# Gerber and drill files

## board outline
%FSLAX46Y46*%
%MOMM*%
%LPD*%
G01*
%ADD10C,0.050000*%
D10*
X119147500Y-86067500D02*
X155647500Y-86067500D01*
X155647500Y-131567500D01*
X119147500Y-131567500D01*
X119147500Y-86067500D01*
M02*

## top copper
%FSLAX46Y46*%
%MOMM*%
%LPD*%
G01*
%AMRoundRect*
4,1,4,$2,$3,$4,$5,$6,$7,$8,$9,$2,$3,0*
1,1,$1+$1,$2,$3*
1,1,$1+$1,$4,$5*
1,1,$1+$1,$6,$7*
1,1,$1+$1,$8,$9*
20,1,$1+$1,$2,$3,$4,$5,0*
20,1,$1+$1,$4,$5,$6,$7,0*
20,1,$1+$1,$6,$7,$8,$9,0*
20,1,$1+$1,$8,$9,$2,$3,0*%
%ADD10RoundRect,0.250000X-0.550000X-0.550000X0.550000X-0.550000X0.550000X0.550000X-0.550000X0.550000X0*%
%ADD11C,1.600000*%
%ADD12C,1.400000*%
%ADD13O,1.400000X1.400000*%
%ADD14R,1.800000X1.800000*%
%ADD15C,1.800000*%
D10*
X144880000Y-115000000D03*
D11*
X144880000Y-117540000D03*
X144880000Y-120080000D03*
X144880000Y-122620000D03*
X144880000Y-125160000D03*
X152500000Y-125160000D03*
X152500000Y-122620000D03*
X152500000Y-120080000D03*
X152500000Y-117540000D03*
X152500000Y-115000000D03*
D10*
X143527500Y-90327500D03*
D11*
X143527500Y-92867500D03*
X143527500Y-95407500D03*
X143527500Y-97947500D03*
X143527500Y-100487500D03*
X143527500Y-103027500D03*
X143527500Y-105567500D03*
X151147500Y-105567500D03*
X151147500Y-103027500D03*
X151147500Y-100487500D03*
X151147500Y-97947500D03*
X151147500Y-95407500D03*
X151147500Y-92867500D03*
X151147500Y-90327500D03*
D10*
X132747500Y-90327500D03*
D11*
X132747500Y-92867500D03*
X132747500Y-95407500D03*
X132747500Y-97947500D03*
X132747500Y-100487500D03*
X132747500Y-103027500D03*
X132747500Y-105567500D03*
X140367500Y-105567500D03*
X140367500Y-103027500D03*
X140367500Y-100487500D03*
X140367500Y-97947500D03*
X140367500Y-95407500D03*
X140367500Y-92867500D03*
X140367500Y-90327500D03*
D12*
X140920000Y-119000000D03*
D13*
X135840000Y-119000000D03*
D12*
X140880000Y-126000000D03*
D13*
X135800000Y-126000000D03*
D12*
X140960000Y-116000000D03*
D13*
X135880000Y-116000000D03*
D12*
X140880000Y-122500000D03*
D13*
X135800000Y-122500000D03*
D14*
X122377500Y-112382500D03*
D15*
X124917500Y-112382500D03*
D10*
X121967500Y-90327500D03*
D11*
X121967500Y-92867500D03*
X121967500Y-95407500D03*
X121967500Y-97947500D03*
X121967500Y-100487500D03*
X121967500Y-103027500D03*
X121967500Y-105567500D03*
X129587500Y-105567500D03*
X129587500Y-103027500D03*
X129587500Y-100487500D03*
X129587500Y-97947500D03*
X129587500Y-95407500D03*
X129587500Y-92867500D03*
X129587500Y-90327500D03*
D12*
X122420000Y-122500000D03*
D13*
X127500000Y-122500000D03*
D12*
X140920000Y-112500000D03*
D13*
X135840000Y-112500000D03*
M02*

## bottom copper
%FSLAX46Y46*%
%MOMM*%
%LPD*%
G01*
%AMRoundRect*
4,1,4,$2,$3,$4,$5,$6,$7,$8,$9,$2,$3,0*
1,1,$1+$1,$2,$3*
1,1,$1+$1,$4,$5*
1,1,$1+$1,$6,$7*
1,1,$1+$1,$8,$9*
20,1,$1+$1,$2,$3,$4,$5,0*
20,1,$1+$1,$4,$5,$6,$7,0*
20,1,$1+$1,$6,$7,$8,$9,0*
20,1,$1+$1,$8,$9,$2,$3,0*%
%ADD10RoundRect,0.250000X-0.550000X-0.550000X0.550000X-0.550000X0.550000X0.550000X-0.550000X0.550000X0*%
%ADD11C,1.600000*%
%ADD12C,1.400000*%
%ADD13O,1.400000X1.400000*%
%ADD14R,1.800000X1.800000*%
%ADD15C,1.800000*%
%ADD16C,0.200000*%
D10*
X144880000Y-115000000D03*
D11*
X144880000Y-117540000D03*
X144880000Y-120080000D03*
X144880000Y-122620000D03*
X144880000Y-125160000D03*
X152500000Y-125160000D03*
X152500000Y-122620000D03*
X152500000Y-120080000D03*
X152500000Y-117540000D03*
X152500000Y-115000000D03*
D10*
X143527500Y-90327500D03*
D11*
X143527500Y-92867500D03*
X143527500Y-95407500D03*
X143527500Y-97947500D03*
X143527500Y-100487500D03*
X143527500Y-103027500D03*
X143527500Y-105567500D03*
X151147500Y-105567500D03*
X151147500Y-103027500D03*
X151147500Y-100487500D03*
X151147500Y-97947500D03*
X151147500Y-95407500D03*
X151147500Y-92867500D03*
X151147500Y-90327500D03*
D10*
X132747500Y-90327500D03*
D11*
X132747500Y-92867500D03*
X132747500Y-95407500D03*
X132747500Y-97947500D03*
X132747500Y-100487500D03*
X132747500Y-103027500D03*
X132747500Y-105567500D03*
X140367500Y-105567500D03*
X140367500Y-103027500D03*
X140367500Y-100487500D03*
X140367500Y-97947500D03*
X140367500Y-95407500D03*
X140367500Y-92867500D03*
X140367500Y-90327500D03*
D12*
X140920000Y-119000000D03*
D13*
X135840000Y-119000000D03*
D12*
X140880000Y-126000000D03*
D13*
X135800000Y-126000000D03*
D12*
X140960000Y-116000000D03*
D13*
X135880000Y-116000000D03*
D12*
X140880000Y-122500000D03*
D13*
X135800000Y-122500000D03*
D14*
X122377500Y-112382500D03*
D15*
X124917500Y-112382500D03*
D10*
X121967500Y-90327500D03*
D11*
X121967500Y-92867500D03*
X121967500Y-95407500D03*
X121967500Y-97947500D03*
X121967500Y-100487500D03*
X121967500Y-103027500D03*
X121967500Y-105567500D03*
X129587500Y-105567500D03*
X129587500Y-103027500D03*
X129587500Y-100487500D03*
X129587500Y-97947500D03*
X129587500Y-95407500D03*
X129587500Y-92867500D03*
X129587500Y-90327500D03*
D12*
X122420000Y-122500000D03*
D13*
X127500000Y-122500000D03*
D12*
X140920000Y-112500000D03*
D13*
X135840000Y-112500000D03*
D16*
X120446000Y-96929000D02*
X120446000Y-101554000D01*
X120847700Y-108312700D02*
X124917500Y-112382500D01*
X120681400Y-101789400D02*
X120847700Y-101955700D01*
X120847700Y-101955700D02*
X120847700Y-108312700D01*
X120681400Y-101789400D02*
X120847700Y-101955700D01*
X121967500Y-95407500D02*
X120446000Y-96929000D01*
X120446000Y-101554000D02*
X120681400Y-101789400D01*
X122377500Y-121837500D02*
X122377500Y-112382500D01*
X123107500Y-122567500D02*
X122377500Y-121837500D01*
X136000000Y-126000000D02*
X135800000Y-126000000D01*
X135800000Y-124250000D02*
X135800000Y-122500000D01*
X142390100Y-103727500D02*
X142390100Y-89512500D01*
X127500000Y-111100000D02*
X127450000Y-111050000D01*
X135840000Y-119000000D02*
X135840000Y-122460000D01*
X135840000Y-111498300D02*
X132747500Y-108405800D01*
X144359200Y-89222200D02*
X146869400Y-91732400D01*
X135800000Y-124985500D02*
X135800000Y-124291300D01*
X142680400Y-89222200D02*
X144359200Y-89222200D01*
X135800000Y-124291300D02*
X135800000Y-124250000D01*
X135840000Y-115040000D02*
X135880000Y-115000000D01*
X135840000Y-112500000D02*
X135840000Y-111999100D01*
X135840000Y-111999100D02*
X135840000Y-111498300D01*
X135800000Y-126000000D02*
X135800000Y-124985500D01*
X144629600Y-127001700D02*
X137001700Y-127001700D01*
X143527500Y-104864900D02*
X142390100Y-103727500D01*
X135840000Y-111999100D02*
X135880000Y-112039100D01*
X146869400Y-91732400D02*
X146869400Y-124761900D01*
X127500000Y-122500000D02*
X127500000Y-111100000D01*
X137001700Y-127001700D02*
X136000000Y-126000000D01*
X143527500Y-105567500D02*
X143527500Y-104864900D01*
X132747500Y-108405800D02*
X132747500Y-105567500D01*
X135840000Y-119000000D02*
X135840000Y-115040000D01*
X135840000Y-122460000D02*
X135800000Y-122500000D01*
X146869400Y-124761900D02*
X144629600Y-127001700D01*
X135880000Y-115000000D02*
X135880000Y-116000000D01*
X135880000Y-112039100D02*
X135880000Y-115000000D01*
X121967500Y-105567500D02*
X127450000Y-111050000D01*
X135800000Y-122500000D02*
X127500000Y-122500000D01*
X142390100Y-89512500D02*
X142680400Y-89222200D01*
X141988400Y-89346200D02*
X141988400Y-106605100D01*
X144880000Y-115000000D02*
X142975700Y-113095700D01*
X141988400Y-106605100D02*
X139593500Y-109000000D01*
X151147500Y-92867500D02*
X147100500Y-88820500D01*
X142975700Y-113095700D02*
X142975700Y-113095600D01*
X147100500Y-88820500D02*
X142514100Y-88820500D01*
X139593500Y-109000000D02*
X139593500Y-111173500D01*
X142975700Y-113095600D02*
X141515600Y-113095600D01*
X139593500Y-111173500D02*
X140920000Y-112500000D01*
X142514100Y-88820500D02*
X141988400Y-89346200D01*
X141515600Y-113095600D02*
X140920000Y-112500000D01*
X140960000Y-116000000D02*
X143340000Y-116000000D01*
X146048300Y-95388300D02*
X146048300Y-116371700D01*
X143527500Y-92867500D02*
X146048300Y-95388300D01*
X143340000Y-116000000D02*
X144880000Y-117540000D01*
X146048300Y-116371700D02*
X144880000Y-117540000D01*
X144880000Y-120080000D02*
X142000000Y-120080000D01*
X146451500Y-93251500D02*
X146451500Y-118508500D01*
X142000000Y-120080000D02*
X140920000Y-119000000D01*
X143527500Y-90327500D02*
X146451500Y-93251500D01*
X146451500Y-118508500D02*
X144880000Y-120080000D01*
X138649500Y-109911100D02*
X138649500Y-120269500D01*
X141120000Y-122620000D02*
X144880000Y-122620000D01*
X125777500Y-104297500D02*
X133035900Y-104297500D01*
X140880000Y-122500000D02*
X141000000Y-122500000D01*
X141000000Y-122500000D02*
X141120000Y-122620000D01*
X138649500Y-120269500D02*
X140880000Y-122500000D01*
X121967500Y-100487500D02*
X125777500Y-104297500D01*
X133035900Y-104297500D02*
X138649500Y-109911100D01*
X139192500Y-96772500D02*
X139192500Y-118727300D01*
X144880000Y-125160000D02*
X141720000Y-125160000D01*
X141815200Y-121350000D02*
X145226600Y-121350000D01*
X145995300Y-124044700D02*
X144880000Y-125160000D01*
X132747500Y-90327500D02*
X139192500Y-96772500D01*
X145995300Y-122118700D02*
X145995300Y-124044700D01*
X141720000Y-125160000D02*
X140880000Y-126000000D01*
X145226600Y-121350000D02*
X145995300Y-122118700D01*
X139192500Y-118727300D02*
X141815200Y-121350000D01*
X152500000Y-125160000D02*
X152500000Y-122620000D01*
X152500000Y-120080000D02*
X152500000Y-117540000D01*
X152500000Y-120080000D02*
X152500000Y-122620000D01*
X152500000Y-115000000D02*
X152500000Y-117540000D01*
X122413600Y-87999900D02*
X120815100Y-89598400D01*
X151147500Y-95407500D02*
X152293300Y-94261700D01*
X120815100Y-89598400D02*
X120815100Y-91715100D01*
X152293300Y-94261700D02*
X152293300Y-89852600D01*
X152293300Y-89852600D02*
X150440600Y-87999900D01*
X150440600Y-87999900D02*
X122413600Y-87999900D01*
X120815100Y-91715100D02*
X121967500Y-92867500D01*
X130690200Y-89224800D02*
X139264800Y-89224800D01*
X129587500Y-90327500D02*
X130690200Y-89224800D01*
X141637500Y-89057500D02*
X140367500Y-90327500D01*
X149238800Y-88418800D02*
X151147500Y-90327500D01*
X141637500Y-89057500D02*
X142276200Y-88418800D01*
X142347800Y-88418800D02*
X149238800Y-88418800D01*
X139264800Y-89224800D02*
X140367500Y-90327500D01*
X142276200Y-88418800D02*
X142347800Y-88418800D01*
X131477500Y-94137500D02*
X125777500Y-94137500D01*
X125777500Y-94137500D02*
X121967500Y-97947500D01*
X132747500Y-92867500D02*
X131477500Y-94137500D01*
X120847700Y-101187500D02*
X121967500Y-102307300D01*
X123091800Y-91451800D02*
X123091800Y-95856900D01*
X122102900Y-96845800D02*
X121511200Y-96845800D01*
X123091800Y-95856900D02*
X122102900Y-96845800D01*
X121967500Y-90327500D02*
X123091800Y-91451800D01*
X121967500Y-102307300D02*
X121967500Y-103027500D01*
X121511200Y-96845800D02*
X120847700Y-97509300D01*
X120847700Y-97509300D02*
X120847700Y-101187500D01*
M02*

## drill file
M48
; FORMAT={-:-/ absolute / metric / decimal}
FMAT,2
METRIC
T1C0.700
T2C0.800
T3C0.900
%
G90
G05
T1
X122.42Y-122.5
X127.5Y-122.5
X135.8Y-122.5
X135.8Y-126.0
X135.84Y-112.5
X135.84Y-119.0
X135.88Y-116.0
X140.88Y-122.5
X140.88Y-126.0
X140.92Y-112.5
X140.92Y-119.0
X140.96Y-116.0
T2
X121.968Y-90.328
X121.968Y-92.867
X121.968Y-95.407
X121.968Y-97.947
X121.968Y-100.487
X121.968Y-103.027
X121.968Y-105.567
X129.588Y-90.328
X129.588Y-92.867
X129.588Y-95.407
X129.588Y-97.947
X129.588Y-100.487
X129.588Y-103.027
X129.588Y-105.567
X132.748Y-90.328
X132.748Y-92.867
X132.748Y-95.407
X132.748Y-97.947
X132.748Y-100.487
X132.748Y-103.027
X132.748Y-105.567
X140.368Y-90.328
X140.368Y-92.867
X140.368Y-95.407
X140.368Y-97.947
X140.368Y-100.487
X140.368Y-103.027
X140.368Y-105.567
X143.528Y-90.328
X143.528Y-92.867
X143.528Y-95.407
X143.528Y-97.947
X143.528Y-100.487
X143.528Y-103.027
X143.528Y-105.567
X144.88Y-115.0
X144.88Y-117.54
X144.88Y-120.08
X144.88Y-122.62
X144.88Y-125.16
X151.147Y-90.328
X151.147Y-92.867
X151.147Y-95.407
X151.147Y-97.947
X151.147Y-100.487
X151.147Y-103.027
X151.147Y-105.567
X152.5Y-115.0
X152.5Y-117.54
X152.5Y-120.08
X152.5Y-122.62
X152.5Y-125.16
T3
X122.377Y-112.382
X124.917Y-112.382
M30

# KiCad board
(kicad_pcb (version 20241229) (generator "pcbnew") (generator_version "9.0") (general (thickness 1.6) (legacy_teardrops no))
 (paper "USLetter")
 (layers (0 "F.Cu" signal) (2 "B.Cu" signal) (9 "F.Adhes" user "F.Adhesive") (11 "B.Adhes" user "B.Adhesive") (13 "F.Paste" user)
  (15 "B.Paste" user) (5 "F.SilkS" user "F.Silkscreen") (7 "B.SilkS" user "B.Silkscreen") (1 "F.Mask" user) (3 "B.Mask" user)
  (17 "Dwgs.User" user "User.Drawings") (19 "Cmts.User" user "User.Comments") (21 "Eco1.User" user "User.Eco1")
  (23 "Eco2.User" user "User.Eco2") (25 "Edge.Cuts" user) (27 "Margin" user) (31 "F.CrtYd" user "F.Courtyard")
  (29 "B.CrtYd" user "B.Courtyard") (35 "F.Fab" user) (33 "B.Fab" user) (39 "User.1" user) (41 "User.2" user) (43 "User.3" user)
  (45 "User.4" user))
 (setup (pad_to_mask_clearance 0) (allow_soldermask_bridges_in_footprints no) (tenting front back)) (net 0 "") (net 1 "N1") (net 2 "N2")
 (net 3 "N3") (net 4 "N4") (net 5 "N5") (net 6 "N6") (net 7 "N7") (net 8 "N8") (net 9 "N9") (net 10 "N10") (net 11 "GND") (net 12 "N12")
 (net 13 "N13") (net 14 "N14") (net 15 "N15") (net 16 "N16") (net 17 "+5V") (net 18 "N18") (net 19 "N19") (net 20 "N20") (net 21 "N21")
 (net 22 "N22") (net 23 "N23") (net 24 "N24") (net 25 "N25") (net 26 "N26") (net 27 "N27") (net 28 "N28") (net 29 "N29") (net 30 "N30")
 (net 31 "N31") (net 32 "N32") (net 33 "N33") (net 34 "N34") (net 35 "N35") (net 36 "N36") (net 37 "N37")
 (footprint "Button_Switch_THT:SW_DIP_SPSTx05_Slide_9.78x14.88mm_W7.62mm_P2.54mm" (layer "F.Cu") (at 144.88 115)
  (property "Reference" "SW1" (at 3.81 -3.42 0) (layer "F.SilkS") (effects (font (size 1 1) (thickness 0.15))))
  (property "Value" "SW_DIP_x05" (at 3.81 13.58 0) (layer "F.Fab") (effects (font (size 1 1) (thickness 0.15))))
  (pad "1" thru_hole roundrect (at 0 0) (size 1.6 1.6) (drill 0.8) (layers "*.Cu" "*.Mask") (remove_unused_layers no)
   (roundrect_rratio 0.15625) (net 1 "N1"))
  (pad "2" thru_hole circle (at 0 2.54) (size 1.6 1.6) (drill 0.8) (layers "*.Cu" "*.Mask") (remove_unused_layers no) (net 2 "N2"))
  (pad "3" thru_hole circle (at 0 5.08) (size 1.6 1.6) (drill 0.8) (layers "*.Cu" "*.Mask") (remove_unused_layers no) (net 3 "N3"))
  (pad "4" thru_hole circle (at 0 7.62) (size 1.6 1.6) (drill 0.8) (layers "*.Cu" "*.Mask") (remove_unused_layers no) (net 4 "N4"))
  (pad "5" thru_hole circle (at 0 10.16) (size 1.6 1.6) (drill 0.8) (layers "*.Cu" "*.Mask") (remove_unused_layers no) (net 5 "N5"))
  (pad "6" thru_hole circle (at 7.62 10.16) (size 1.6 1.6) (drill 0.8) (layers "*.Cu" "*.Mask") (remove_unused_layers no) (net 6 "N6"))
  (pad "7" thru_hole circle (at 7.62 7.62) (size 1.6 1.6) (drill 0.8) (layers "*.Cu" "*.Mask") (remove_unused_layers no) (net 6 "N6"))
  (pad "8" thru_hole circle (at 7.62 5.08) (size 1.6 1.6) (drill 0.8) (layers "*.Cu" "*.Mask") (remove_unused_layers no) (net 6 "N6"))
  (pad "9" thru_hole circle (at 7.62 2.54) (size 1.6 1.6) (drill 0.8) (layers "*.Cu" "*.Mask") (remove_unused_layers no) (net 6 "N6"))
  (pad "10" thru_hole circle (at 7.62 0) (size 1.6 1.6) (drill 0.8) (layers "*.Cu" "*.Mask") (remove_unused_layers no) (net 6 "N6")))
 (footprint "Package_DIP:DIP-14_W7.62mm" (layer "F.Cu") (at 143.5275 90.3275)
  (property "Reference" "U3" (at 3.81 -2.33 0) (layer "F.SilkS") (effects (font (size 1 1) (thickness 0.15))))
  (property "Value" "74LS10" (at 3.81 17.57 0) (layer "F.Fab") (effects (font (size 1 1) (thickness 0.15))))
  (pad "1" thru_hole roundrect (at 0 0) (size 1.6 1.6) (drill 0.8) (layers "*.Cu" "*.Mask") (remove_unused_layers no)
   (roundrect_rratio 0.15625) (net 3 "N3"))
  (pad "2" thru_hole circle (at 0 2.54) (size 1.6 1.6) (drill 0.8) (layers "*.Cu" "*.Mask") (remove_unused_layers no) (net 2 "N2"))
  (pad "3" thru_hole circle (at 0 5.08) (size 1.6 1.6) (drill 0.8) (layers "*.Cu" "*.Mask") (remove_unused_layers no) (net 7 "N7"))
  (pad "4" thru_hole circle (at 0 7.62) (size 1.6 1.6) (drill 0.8) (layers "*.Cu" "*.Mask") (remove_unused_layers no) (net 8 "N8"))
  (pad "5" thru_hole circle (at 0 10.16) (size 1.6 1.6) (drill 0.8) (layers "*.Cu" "*.Mask") (remove_unused_layers no) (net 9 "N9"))
  (pad "6" thru_hole circle (at 0 12.7) (size 1.6 1.6) (drill 0.8) (layers "*.Cu" "*.Mask") (remove_unused_layers no) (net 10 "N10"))
  (pad "7" thru_hole circle (at 0 15.24) (size 1.6 1.6) (drill 0.8) (layers "*.Cu" "*.Mask") (remove_unused_layers no) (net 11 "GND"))
  (pad "8" thru_hole circle (at 7.62 15.24) (size 1.6 1.6) (drill 0.8) (layers "*.Cu" "*.Mask") (remove_unused_layers no) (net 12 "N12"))
  (pad "9" thru_hole circle (at 7.62 12.7) (size 1.6 1.6) (drill 0.8) (layers "*.Cu" "*.Mask") (remove_unused_layers no) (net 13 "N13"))
  (pad "10" thru_hole circle (at 7.62 10.16) (size 1.6 1.6) (drill 0.8) (layers "*.Cu" "*.Mask") (remove_unused_layers no) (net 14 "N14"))
  (pad "11" thru_hole circle (at 7.62 7.62) (size 1.6 1.6) (drill 0.8) (layers "*.Cu" "*.Mask") (remove_unused_layers no) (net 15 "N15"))
  (pad "12" thru_hole circle (at 7.62 5.08) (size 1.6 1.6) (drill 0.8) (layers "*.Cu" "*.Mask") (remove_unused_layers no) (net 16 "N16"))
  (pad "13" thru_hole circle (at 7.62 2.54) (size 1.6 1.6) (drill 0.8) (layers "*.Cu" "*.Mask") (remove_unused_layers no) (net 1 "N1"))
  (pad "14" thru_hole circle (at 7.62 0) (size 1.6 1.6) (drill 0.8) (layers "*.Cu" "*.Mask") (remove_unused_layers no) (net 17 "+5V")))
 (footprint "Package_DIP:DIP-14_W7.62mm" (layer "F.Cu") (at 132.7475 90.3275)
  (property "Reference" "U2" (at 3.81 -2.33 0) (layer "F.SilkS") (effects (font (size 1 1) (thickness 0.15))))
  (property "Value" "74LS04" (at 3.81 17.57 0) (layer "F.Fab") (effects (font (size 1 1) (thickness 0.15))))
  (pad "1" thru_hole roundrect (at 0 0) (size 1.6 1.6) (drill 0.8) (layers "*.Cu" "*.Mask") (remove_unused_layers no)
   (roundrect_rratio 0.15625) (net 5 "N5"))
  (pad "2" thru_hole circle (at 0 2.54) (size 1.6 1.6) (drill 0.8) (layers "*.Cu" "*.Mask") (remove_unused_layers no) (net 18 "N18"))
  (pad "3" thru_hole circle (at 0 5.08) (size 1.6 1.6) (drill 0.8) (layers "*.Cu" "*.Mask") (remove_unused_layers no) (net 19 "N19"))
  (pad "4" thru_hole circle (at 0 7.62) (size 1.6 1.6) (drill 0.8) (layers "*.Cu" "*.Mask") (remove_unused_layers no) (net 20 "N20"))
  (pad "5" thru_hole circle (at 0 10.16) (size 1.6 1.6) (drill 0.8) (layers "*.Cu" "*.Mask") (remove_unused_layers no) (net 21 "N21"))
  (pad "6" thru_hole circle (at 0 12.7) (size 1.6 1.6) (drill 0.8) (layers "*.Cu" "*.Mask") (remove_unused_layers no) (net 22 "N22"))
  (pad "7" thru_hole circle (at 0 15.24) (size 1.6 1.6) (drill 0.8) (layers "*.Cu" "*.Mask") (remove_unused_layers no) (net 11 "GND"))
  (pad "8" thru_hole circle (at 7.62 15.24) (size 1.6 1.6) (drill 0.8) (layers "*.Cu" "*.Mask") (remove_unused_layers no) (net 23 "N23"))
  (pad "9" thru_hole circle (at 7.62 12.7) (size 1.6 1.6) (drill 0.8) (layers "*.Cu" "*.Mask") (remove_unused_layers no) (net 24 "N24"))
  (pad "10" thru_hole circle (at 7.62 10.16) (size 1.6 1.6) (drill 0.8) (layers "*.Cu" "*.Mask") (remove_unused_layers no) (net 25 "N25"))
  (pad "11" thru_hole circle (at 7.62 7.62) (size 1.6 1.6) (drill 0.8) (layers "*.Cu" "*.Mask") (remove_unused_layers no) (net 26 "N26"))
  (pad "12" thru_hole circle (at 7.62 5.08) (size 1.6 1.6) (drill 0.8) (layers "*.Cu" "*.Mask") (remove_unused_layers no) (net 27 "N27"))
  (pad "13" thru_hole circle (at 7.62 2.54) (size 1.6 1.6) (drill 0.8) (layers "*.Cu" "*.Mask") (remove_unused_layers no) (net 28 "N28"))
  (pad "14" thru_hole circle (at 7.62 0) (size 1.6 1.6) (drill 0.8) (layers "*.Cu" "*.Mask") (remove_unused_layers no) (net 17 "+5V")))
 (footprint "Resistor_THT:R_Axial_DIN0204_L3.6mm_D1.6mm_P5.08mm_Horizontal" (layer "F.Cu") (at 140.92 119 180)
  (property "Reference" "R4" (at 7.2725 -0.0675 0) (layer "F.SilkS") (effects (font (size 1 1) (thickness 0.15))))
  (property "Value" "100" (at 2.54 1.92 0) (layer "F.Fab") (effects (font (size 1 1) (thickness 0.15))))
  (pad "1" thru_hole circle (at 0 0 180) (size 1.4 1.4) (drill 0.7) (layers "*.Cu" "*.Mask") (remove_unused_layers no) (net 3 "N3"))
  (pad "2" thru_hole oval (at 5.08 0 180) (size 1.4 1.4) (drill 0.7) (layers "*.Cu" "*.Mask") (remove_unused_layers no) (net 11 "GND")))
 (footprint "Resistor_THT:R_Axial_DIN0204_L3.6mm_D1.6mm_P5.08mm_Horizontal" (layer "F.Cu") (at 140.88 126 180)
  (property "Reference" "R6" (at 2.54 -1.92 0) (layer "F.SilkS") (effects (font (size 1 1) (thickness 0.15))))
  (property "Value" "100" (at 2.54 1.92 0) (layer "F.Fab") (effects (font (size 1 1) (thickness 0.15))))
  (pad "1" thru_hole circle (at 0 0 180) (size 1.4 1.4) (drill 0.7) (layers "*.Cu" "*.Mask") (remove_unused_layers no) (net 5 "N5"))
  (pad "2" thru_hole oval (at 5.08 0 180) (size 1.4 1.4) (drill 0.7) (layers "*.Cu" "*.Mask") (remove_unused_layers no) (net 11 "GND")))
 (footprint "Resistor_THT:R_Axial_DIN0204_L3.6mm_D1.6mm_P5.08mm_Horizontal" (layer "F.Cu") (at 140.96 116 180)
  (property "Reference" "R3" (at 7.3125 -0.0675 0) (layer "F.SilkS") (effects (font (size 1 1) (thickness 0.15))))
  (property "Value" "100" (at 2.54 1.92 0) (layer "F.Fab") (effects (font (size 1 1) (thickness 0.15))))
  (pad "1" thru_hole circle (at 0 0 180) (size 1.4 1.4) (drill 0.7) (layers "*.Cu" "*.Mask") (remove_unused_layers no) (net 2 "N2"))
  (pad "2" thru_hole oval (at 5.08 0 180) (size 1.4 1.4) (drill 0.7) (layers "*.Cu" "*.Mask") (remove_unused_layers no) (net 11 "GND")))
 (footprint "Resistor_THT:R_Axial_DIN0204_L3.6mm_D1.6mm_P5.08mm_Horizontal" (layer "F.Cu") (at 140.88 122.5 180)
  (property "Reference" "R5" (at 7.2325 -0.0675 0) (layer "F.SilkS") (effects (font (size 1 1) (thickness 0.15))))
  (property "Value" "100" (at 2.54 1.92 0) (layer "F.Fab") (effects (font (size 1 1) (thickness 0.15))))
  (pad "1" thru_hole circle (at 0 0 180) (size 1.4 1.4) (drill 0.7) (layers "*.Cu" "*.Mask") (remove_unused_layers no) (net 4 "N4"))
  (pad "2" thru_hole oval (at 5.08 0 180) (size 1.4 1.4) (drill 0.7) (layers "*.Cu" "*.Mask") (remove_unused_layers no) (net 11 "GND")))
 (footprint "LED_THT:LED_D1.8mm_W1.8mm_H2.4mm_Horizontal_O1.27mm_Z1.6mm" (layer "F.Cu") (at 122.3775 112.3825)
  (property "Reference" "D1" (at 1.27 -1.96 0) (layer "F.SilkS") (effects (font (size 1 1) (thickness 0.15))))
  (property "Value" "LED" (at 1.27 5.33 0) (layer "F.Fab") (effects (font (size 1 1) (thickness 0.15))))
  (pad "1" thru_hole rect (at 0 0) (size 1.8 1.8) (drill 0.9) (layers "*.Cu" "*.Mask") (remove_unused_layers no) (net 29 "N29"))
  (pad "2" thru_hole circle (at 2.54 0) (size 1.8 1.8) (drill 0.9) (layers "*.Cu" "*.Mask") (remove_unused_layers no) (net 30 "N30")))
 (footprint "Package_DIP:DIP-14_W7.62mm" (layer "F.Cu") (at 121.9675 90.3275)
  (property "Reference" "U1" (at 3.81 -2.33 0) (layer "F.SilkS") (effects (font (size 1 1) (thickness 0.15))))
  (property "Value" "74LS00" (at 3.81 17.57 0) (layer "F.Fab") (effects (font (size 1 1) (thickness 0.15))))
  (pad "1" thru_hole roundrect (at 0 0) (size 1.6 1.6) (drill 0.8) (layers "*.Cu" "*.Mask") (remove_unused_layers no)
   (roundrect_rratio 0.15625) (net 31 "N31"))
  (pad "2" thru_hole circle (at 0 2.54) (size 1.6 1.6) (drill 0.8) (layers "*.Cu" "*.Mask") (remove_unused_layers no) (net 16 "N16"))
  (pad "3" thru_hole circle (at 0 5.08) (size 1.6 1.6) (drill 0.8) (layers "*.Cu" "*.Mask") (remove_unused_layers no) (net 30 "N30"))
  (pad "4" thru_hole circle (at 0 7.62) (size 1.6 1.6) (drill 0.8) (layers "*.Cu" "*.Mask") (remove_unused_layers no) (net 18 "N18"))
  (pad "5" thru_hole circle (at 0 10.16) (size 1.6 1.6) (drill 0.8) (layers "*.Cu" "*.Mask") (remove_unused_layers no) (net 4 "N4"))
  (pad "6" thru_hole circle (at 0 12.7) (size 1.6 1.6) (drill 0.8) (layers "*.Cu" "*.Mask") (remove_unused_layers no) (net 31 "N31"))
  (pad "7" thru_hole circle (at 0 15.24) (size 1.6 1.6) (drill 0.8) (layers "*.Cu" "*.Mask") (remove_unused_layers no) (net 11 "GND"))
  (pad "8" thru_hole circle (at 7.62 15.24) (size 1.6 1.6) (drill 0.8) (layers "*.Cu" "*.Mask") (remove_unused_layers no) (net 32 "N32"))
  (pad "9" thru_hole circle (at 7.62 12.7) (size 1.6 1.6) (drill 0.8) (layers "*.Cu" "*.Mask") (remove_unused_layers no) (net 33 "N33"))
  (pad "10" thru_hole circle (at 7.62 10.16) (size 1.6 1.6) (drill 0.8) (layers "*.Cu" "*.Mask") (remove_unused_layers no) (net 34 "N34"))
  (pad "11" thru_hole circle (at 7.62 7.62) (size 1.6 1.6) (drill 0.8) (layers "*.Cu" "*.Mask") (remove_unused_layers no) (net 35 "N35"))
  (pad "12" thru_hole circle (at 7.62 5.08) (size 1.6 1.6) (drill 0.8) (layers "*.Cu" "*.Mask") (remove_unused_layers no) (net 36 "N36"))
  (pad "13" thru_hole circle (at 7.62 2.54) (size 1.6 1.6) (drill 0.8) (layers "*.Cu" "*.Mask") (remove_unused_layers no) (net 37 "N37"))
  (pad "14" thru_hole circle (at 7.62 0) (size 1.6 1.6) (drill 0.8) (layers "*.Cu" "*.Mask") (remove_unused_layers no) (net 17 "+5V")))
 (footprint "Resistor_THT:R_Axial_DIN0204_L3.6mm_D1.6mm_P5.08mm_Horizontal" (layer "F.Cu") (at 122.42 122.5)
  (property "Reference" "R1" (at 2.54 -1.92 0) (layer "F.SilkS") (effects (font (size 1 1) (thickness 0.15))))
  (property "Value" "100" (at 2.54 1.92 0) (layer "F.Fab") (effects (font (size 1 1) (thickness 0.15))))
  (pad "1" thru_hole circle (at 0 0) (size 1.4 1.4) (drill 0.7) (layers "*.Cu" "*.Mask") (remove_unused_layers no) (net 29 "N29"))
  (pad "2" thru_hole oval (at 5.08 0) (size 1.4 1.4) (drill 0.7) (layers "*.Cu" "*.Mask") (remove_unused_layers no) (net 11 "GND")))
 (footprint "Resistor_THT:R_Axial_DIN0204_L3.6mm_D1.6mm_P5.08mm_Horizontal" (layer "F.Cu") (at 140.92 112.5 180)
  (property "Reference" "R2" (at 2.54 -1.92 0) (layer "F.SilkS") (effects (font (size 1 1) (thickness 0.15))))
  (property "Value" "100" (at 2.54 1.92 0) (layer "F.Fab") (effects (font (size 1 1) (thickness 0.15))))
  (pad "1" thru_hole circle (at 0 0 180) (size 1.4 1.4) (drill 0.7) (layers "*.Cu" "*.Mask") (remove_unused_layers no) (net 1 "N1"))
  (pad "2" thru_hole oval (at 5.08 0 180) (size 1.4 1.4) (drill 0.7) (layers "*.Cu" "*.Mask") (remove_unused_layers no) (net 11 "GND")))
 (gr_rect (start 119.1475 86.0675) (end 155.6475 131.5675) (stroke (width 0.05) (type default)) (fill no) (layer "Edge.Cuts"))
 (segment (start 120.446 96.929) (end 120.446 101.554) (width 0.2) (layer "B.Cu") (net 30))
 (segment (start 120.8477 108.3127) (end 124.9175 112.3825) (width 0.2) (layer "B.Cu") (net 30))
 (segment (start 120.6814 101.7894) (end 120.8477 101.9557) (width 0.2) (layer "B.Cu") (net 30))
 (segment (start 120.8477 101.9557) (end 120.8477 108.3127) (width 0.2) (layer "B.Cu") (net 30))
 (segment (start 120.6814 101.7894) (end 120.8477 101.9557) (width 0.2) (layer "B.Cu") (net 30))
 (segment (start 121.9675 95.4075) (end 120.446 96.929) (width 0.2) (layer "B.Cu") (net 30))
 (segment (start 120.446 101.554) (end 120.6814 101.7894) (width 0.2) (layer "B.Cu") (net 30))
 (segment (start 122.3775 121.8375) (end 122.3775 112.3825) (width 0.2) (layer "B.Cu") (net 29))
 (segment (start 123.1075 122.5675) (end 122.3775 121.8375) (width 0.2) (layer "B.Cu") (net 29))
 (segment (start 136 126) (end 135.8 126) (width 0.2) (layer "B.Cu") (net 11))
 (segment (start 135.8 124.25) (end 135.8 122.5) (width 0.2) (layer "B.Cu") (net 11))
 (segment (start 142.3901 103.7275) (end 142.3901 89.5125) (width 0.2) (layer "B.Cu") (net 11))
 (segment (start 127.5 111.1) (end 127.45 111.05) (width 0.2) (layer "B.Cu") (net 11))
 (segment (start 135.84 119) (end 135.84 122.46) (width 0.2) (layer "B.Cu") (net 11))
 (segment (start 135.84 111.4983) (end 132.7475 108.4058) (width 0.2) (layer "B.Cu") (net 11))
 (segment (start 144.3592 89.2222) (end 146.8694 91.7324) (width 0.2) (layer "B.Cu") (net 11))
 (segment (start 135.8 124.9855) (end 135.8 124.2913) (width 0.2) (layer "B.Cu") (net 11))
 (segment (start 142.6804 89.2222) (end 144.3592 89.2222) (width 0.2) (layer "B.Cu") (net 11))
 (segment (start 135.8 124.2913) (end 135.8 124.25) (width 0.2) (layer "B.Cu") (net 11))
 (segment (start 135.84 115.04) (end 135.88 115) (width 0.2) (layer "B.Cu") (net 11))
 (segment (start 135.84 112.5) (end 135.84 111.9991) (width 0.2) (layer "B.Cu") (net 11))
 (segment (start 135.84 111.9991) (end 135.84 111.4983) (width 0.2) (layer "B.Cu") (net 11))
 (segment (start 135.8 126) (end 135.8 124.9855) (width 0.2) (layer "B.Cu") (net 11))
 (segment (start 144.6296 127.0017) (end 137.0017 127.0017) (width 0.2) (layer "B.Cu") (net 11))
 (segment (start 143.5275 104.8649) (end 142.3901 103.7275) (width 0.2) (layer "B.Cu") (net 11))
 (segment (start 135.84 111.9991) (end 135.88 112.0391) (width 0.2) (layer "B.Cu") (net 11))
 (segment (start 146.8694 91.7324) (end 146.8694 124.7619) (width 0.2) (layer "B.Cu") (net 11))
 (segment (start 127.5 122.5) (end 127.5 111.1) (width 0.2) (layer "B.Cu") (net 11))
 (segment (start 137.0017 127.0017) (end 136 126) (width 0.2) (layer "B.Cu") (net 11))
 (segment (start 143.5275 105.5675) (end 143.5275 104.8649) (width 0.2) (layer "B.Cu") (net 11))
 (segment (start 132.7475 108.4058) (end 132.7475 105.5675) (width 0.2) (layer "B.Cu") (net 11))
 (segment (start 135.84 119) (end 135.84 115.04) (width 0.2) (layer "B.Cu") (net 11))
 (segment (start 135.84 122.46) (end 135.8 122.5) (width 0.2) (layer "B.Cu") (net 11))
 (segment (start 146.8694 124.7619) (end 144.6296 127.0017) (width 0.2) (layer "B.Cu") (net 11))
 (segment (start 135.88 115) (end 135.88 116) (width 0.2) (layer "B.Cu") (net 11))
 (segment (start 135.88 112.0391) (end 135.88 115) (width 0.2) (layer "B.Cu") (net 11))
 (segment (start 121.9675 105.5675) (end 127.45 111.05) (width 0.2) (layer "B.Cu") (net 11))
 (segment (start 135.8 122.5) (end 127.5 122.5) (width 0.2) (layer "B.Cu") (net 11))
 (segment (start 142.3901 89.5125) (end 142.6804 89.2222) (width 0.2) (layer "B.Cu") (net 11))
 (segment (start 141.9884 89.3462) (end 141.9884 106.6051) (width 0.2) (layer "B.Cu") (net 1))
 (segment (start 144.88 115) (end 142.9757 113.0957) (width 0.2) (layer "B.Cu") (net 1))
 (segment (start 141.9884 106.6051) (end 139.5935 109) (width 0.2) (layer "B.Cu") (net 1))
 (segment (start 151.1475 92.8675) (end 147.1005 88.8205) (width 0.2) (layer "B.Cu") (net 1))
 (segment (start 142.9757 113.0957) (end 142.9757 113.0956) (width 0.2) (layer "B.Cu") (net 1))
 (segment (start 147.1005 88.8205) (end 142.5141 88.8205) (width 0.2) (layer "B.Cu") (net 1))
 (segment (start 139.5935 109) (end 139.5935 111.1735) (width 0.2) (layer "B.Cu") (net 1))
 (segment (start 142.9757 113.0956) (end 141.5156 113.0956) (width 0.2) (layer "B.Cu") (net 1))
 (segment (start 139.5935 111.1735) (end 140.92 112.5) (width 0.2) (layer "B.Cu") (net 1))
 (segment (start 142.5141 88.8205) (end 141.9884 89.3462) (width 0.2) (layer "B.Cu") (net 1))
 (segment (start 141.5156 113.0956) (end 140.92 112.5) (width 0.2) (layer "B.Cu") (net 1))
 (segment (start 140.96 116) (end 143.34 116) (width 0.2) (layer "B.Cu") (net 2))
 (segment (start 146.0483 95.3883) (end 146.0483 116.3717) (width 0.2) (layer "B.Cu") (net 2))
 (segment (start 143.5275 92.8675) (end 146.0483 95.3883) (width 0.2) (layer "B.Cu") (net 2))
 (segment (start 143.34 116) (end 144.88 117.54) (width 0.2) (layer "B.Cu") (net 2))
 (segment (start 146.0483 116.3717) (end 144.88 117.54) (width 0.2) (layer "B.Cu") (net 2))
 (segment (start 144.88 120.08) (end 142 120.08) (width 0.2) (layer "B.Cu") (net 3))
 (segment (start 146.4515 93.2515) (end 146.4515 118.5085) (width 0.2) (layer "B.Cu") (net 3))
 (segment (start 142 120.08) (end 140.92 119) (width 0.2) (layer "B.Cu") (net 3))
 (segment (start 143.5275 90.3275) (end 146.4515 93.2515) (width 0.2) (layer "B.Cu") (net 3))
 (segment (start 146.4515 118.5085) (end 144.88 120.08) (width 0.2) (layer "B.Cu") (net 3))
 (segment (start 138.6495 109.9111) (end 138.6495 120.2695) (width 0.2) (layer "B.Cu") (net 4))
 (segment (start 141.12 122.62) (end 144.88 122.62) (width 0.2) (layer "B.Cu") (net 4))
 (segment (start 125.7775 104.2975) (end 133.0359 104.2975) (width 0.2) (layer "B.Cu") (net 4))
 (segment (start 140.88 122.5) (end 141 122.5) (width 0.2) (layer "B.Cu") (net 4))
 (segment (start 141 122.5) (end 141.12 122.62) (width 0.2) (layer "B.Cu") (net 4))
 (segment (start 138.6495 120.2695) (end 140.88 122.5) (width 0.2) (layer "B.Cu") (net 4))
 (segment (start 121.9675 100.4875) (end 125.7775 104.2975) (width 0.2) (layer "B.Cu") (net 4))
 (segment (start 133.0359 104.2975) (end 138.6495 109.9111) (width 0.2) (layer "B.Cu") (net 4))
 (segment (start 139.1925 96.7725) (end 139.1925 118.7273) (width 0.2) (layer "B.Cu") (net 5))
 (segment (start 144.88 125.16) (end 141.72 125.16) (width 0.2) (layer "B.Cu") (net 5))
 (segment (start 141.8152 121.35) (end 145.2266 121.35) (width 0.2) (layer "B.Cu") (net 5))
 (segment (start 145.9953 124.0447) (end 144.88 125.16) (width 0.2) (layer "B.Cu") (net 5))
 (segment (start 132.7475 90.3275) (end 139.1925 96.7725) (width 0.2) (layer "B.Cu") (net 5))
 (segment (start 145.9953 122.1187) (end 145.9953 124.0447) (width 0.2) (layer "B.Cu") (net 5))
 (segment (start 141.72 125.16) (end 140.88 126) (width 0.2) (layer "B.Cu") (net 5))
 (segment (start 145.2266 121.35) (end 145.9953 122.1187) (width 0.2) (layer "B.Cu") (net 5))
 (segment (start 139.1925 118.7273) (end 141.8152 121.35) (width 0.2) (layer "B.Cu") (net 5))
 (segment (start 152.5 125.16) (end 152.5 122.62) (width 0.2) (layer "B.Cu") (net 6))
 (segment (start 152.5 120.08) (end 152.5 117.54) (width 0.2) (layer "B.Cu") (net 6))
 (segment (start 152.5 120.08) (end 152.5 122.62) (width 0.2) (layer "B.Cu") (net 6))
 (segment (start 152.5 115) (end 152.5 117.54) (width 0.2) (layer "B.Cu") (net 6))
 (segment (start 122.4136 87.9999) (end 120.8151 89.5984) (width 0.2) (layer "B.Cu") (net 16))
 (segment (start 151.1475 95.4075) (end 152.2933 94.2617) (width 0.2) (layer "B.Cu") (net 16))
 (segment (start 120.8151 89.5984) (end 120.8151 91.7151) (width 0.2) (layer "B.Cu") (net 16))
 (segment (start 152.2933 94.2617) (end 152.2933 89.8526) (width 0.2) (layer "B.Cu") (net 16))
 (segment (start 152.2933 89.8526) (end 150.4406 87.9999) (width 0.2) (layer "B.Cu") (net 16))
 (segment (start 150.4406 87.9999) (end 122.4136 87.9999) (width 0.2) (layer "B.Cu") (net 16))
 (segment (start 120.8151 91.7151) (end 121.9675 92.8675) (width 0.2) (layer "B.Cu") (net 16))
 (segment (start 130.6902 89.2248) (end 139.2648 89.2248) (width 0.2) (layer "B.Cu") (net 17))
 (segment (start 129.5875 90.3275) (end 130.6902 89.2248) (width 0.2) (layer "B.Cu") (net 17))
 (segment (start 141.6375 89.0575) (end 140.3675 90.3275) (width 0.2) (layer "B.Cu") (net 17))
 (segment (start 149.2388 88.4188) (end 151.1475 90.3275) (width 0.2) (layer "B.Cu") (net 17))
 (segment (start 141.6375 89.0575) (end 142.2762 88.4188) (width 0.2) (layer "B.Cu") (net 17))
 (segment (start 142.3478 88.4188) (end 149.2388 88.4188) (width 0.2) (layer "B.Cu") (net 17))
 (segment (start 139.2648 89.2248) (end 140.3675 90.3275) (width 0.2) (layer "B.Cu") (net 17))
 (segment (start 142.2762 88.4188) (end 142.3478 88.4188) (width 0.2) (layer "B.Cu") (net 17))
 (segment (start 131.4775 94.1375) (end 125.7775 94.1375) (width 0.2) (layer "B.Cu") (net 18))
 (segment (start 125.7775 94.1375) (end 121.9675 97.9475) (width 0.2) (layer "B.Cu") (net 18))
 (segment (start 132.7475 92.8675) (end 131.4775 94.1375) (width 0.2) (layer "B.Cu") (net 18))
 (segment (start 120.8477 101.1875) (end 121.9675 102.3073) (width 0.2) (layer "B.Cu") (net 31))
 (segment (start 123.0918 91.4518) (end 123.0918 95.8569) (width 0.2) (layer "B.Cu") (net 31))
 (segment (start 122.1029 96.8458) (end 121.5112 96.8458) (width 0.2) (layer "B.Cu") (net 31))
 (segment (start 123.0918 95.8569) (end 122.1029 96.8458) (width 0.2) (layer "B.Cu") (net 31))
 (segment (start 121.9675 90.3275) (end 123.0918 91.4518) (width 0.2) (layer "B.Cu") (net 31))
 (segment (start 121.9675 102.3073) (end 121.9675 103.0275) (width 0.2) (layer "B.Cu") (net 31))
 (segment (start 121.5112 96.8458) (end 120.8477 97.5093) (width 0.2) (layer "B.Cu") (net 31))
 (segment (start 120.8477 97.5093) (end 120.8477 101.1875) (width 0.2) (layer "B.Cu") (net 31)))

